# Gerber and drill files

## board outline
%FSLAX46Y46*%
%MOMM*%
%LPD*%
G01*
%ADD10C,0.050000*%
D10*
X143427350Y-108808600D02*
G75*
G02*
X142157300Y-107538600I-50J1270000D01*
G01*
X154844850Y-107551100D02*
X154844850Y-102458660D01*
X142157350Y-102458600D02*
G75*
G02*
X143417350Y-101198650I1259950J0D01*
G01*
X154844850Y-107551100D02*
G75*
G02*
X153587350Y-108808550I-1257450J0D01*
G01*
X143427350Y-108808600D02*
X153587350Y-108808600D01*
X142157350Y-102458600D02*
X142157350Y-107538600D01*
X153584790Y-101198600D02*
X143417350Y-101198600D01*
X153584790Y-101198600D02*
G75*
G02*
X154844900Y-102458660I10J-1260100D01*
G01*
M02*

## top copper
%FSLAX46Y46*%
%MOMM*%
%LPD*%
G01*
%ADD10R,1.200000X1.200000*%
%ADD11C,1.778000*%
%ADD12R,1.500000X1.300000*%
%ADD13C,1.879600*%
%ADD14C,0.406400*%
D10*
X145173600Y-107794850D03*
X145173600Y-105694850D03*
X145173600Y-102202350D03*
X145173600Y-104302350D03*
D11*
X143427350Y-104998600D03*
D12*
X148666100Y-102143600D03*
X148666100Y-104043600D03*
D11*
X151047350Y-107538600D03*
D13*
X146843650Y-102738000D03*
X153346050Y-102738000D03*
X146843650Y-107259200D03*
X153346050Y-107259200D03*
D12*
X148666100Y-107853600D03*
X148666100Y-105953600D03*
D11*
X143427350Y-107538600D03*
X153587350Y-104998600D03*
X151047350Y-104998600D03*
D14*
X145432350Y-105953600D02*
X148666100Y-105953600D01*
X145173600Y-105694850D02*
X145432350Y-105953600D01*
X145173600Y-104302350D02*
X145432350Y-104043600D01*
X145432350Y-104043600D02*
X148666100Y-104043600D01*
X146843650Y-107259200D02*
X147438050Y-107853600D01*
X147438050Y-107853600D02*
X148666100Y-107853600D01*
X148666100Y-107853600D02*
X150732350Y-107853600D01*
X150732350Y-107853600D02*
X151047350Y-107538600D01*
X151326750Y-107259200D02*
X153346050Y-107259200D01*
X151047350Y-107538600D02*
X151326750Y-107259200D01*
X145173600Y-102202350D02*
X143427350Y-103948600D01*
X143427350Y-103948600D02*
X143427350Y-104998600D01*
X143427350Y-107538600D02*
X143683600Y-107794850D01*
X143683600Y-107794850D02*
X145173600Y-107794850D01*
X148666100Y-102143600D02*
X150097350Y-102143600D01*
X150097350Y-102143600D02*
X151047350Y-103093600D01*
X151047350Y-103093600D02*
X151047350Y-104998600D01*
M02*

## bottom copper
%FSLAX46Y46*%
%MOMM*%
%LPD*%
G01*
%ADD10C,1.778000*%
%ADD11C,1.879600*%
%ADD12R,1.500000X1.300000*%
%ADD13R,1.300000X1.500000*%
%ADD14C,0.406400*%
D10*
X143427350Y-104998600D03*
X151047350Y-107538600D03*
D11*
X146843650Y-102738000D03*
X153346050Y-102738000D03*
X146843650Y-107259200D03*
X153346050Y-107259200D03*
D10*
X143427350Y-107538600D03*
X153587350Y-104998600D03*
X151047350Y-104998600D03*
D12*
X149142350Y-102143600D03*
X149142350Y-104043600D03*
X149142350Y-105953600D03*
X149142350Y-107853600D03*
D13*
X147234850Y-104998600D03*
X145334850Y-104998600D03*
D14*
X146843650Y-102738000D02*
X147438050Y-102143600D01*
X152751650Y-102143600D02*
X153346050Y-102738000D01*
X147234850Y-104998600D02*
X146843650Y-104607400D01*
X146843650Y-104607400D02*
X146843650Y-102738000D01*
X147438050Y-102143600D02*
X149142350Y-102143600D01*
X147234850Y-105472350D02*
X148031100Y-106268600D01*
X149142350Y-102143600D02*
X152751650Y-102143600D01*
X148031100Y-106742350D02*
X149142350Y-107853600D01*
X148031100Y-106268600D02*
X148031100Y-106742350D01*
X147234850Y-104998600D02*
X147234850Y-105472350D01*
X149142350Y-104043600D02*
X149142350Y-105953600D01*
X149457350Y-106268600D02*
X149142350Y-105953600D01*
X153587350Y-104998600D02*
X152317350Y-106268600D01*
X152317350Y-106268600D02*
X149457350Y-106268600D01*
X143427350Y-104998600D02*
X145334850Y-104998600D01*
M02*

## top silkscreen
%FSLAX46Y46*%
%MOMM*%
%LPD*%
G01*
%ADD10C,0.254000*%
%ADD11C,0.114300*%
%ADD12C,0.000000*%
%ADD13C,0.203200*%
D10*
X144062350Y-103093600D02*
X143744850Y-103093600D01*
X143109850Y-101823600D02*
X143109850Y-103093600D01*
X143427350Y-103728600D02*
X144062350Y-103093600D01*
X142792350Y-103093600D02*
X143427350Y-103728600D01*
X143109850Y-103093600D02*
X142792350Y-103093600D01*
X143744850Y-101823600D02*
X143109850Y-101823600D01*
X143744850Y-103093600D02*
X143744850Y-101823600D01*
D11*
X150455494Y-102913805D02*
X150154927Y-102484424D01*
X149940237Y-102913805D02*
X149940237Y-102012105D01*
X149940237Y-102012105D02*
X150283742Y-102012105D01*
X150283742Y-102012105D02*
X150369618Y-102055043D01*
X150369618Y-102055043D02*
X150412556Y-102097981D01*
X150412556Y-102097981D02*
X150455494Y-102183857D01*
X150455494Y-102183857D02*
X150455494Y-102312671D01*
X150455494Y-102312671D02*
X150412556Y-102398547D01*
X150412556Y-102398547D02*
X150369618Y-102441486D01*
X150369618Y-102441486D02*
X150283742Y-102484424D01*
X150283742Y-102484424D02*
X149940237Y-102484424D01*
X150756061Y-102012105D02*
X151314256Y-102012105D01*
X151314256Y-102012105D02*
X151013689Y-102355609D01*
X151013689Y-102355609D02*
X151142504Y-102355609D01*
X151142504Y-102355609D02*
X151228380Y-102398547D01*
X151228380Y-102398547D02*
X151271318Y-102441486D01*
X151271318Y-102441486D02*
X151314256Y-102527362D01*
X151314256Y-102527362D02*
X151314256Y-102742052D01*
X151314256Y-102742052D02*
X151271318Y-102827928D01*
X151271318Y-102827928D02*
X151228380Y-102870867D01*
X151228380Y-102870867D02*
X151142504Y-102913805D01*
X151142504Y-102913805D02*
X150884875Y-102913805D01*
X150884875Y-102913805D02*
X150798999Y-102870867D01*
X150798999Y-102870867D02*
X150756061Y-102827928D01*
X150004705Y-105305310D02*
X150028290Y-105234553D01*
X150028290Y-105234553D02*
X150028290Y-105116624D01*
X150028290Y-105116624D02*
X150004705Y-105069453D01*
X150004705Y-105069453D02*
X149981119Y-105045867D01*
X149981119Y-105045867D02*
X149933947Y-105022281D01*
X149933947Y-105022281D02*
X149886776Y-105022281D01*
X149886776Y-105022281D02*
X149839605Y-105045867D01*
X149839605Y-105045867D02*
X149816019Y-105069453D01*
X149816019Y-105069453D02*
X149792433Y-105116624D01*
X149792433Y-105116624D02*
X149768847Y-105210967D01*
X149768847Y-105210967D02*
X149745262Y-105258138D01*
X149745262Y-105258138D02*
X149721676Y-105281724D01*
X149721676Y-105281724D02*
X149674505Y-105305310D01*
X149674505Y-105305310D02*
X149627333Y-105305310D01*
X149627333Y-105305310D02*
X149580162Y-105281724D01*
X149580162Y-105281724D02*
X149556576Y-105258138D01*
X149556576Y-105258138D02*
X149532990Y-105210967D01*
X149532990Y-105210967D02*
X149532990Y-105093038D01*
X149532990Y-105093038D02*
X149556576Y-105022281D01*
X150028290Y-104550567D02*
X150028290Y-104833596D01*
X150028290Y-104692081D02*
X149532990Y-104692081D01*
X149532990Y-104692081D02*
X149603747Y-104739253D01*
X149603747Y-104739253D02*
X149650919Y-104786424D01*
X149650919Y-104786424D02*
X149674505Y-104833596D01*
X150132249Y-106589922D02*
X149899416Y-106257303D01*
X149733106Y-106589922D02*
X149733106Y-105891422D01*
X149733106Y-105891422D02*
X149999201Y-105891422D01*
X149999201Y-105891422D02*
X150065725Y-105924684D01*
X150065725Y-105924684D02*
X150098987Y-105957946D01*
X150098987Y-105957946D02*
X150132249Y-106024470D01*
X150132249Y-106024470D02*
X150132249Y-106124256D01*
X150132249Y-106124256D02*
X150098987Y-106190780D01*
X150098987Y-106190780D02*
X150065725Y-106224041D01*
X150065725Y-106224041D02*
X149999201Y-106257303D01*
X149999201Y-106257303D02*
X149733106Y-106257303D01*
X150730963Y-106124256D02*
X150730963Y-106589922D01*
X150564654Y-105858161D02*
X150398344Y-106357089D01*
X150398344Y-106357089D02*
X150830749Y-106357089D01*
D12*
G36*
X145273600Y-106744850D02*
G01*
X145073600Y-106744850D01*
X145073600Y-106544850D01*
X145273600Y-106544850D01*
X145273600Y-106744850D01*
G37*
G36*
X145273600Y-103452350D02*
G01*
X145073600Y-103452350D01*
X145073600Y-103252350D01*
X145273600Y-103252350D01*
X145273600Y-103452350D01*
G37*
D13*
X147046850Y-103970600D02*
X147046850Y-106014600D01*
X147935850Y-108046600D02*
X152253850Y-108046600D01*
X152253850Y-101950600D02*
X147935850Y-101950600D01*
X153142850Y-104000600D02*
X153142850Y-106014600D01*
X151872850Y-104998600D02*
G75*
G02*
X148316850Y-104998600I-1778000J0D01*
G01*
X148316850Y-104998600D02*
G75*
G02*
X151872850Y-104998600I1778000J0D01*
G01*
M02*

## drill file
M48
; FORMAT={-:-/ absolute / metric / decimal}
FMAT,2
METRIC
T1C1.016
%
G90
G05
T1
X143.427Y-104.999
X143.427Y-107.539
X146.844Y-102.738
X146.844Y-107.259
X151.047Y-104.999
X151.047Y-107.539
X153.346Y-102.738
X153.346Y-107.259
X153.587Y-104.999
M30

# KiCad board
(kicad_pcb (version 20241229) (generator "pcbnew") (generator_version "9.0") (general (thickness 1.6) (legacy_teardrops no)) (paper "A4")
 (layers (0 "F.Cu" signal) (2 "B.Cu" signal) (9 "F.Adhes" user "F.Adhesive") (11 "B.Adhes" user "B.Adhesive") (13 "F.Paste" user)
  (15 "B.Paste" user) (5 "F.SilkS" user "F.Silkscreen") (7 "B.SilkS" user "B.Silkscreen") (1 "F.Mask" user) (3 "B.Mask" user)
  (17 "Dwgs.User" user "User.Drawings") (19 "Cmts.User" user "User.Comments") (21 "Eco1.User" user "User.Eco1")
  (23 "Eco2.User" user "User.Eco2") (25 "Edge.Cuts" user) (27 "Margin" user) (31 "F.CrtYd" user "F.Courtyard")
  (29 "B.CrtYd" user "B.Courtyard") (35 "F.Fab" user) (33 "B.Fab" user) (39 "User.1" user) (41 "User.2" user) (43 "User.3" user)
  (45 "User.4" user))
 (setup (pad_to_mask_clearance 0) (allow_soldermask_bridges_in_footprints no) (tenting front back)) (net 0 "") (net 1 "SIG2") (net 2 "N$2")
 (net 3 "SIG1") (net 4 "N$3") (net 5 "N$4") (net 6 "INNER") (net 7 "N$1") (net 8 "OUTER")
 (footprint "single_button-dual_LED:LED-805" (layer "F.Cu") (at 145.1736 106.74485)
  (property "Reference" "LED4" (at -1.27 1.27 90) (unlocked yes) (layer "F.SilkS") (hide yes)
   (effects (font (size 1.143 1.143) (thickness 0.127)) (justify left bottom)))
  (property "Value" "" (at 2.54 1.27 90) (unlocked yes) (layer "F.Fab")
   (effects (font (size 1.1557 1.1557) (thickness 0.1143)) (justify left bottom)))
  (fp_poly (pts (xy -0.1 0) (xy 0.1 0) (xy 0.1 -0.2) (xy -0.1 -0.2)) (stroke (width 0) (type default)) (fill yes) (layer "F.SilkS"))
  (pad "A" smd rect (at 0 1.05) (size 1.2 1.2) (layers "F.Cu" "F.Mask" "F.Paste") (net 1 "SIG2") (solder_mask_margin 0.0508)
   (solder_paste_margin 0) (thermal_bridge_angle 0))
  (pad "C" smd rect (at 0 -1.05) (size 1.2 1.2) (layers "F.Cu" "F.Mask" "F.Paste") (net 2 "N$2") (solder_mask_margin 0.0508)
   (solder_paste_margin 0) (thermal_bridge_angle 0)))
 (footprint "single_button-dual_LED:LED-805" (layer "F.Cu") (at 145.1736 103.25235 180)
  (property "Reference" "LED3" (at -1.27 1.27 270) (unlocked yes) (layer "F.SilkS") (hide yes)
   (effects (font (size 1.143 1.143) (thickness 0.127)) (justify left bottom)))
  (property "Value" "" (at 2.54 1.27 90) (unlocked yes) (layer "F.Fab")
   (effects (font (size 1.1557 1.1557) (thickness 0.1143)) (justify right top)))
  (fp_poly (pts (xy -0.1 0) (xy 0.1 0) (xy 0.1 -0.2) (xy -0.1 -0.2)) (stroke (width 0) (type default)) (fill yes) (layer "F.SilkS"))
  (pad "A" smd rect (at 0 1.05 180) (size 1.2 1.2) (layers "F.Cu" "F.Mask" "F.Paste") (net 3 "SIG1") (solder_mask_margin 0.0508)
   (solder_paste_margin 0) (thermal_bridge_angle 0))
  (pad "C" smd rect (at 0 -1.05 180) (size 1.2 1.2) (layers "F.Cu" "F.Mask" "F.Paste") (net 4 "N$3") (solder_mask_margin 0.0508)
   (solder_paste_margin 0) (thermal_bridge_angle 0)))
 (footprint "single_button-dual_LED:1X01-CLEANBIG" (layer "F.Cu") (at 143.42735 104.9986)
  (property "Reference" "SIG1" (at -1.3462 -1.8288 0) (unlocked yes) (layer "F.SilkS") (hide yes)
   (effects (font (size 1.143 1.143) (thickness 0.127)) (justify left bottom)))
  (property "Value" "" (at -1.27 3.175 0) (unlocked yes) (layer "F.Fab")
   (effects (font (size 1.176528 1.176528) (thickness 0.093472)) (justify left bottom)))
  (pad "1" thru_hole circle (at 0 0) (size 1.778 1.778) (drill 1.016) (layers "*.Cu" "*.Mask") (remove_unused_layers no) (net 3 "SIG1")
   (solder_mask_margin 0.0508) (thermal_bridge_angle 0)))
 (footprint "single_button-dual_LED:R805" (layer "F.Cu") (at 148.6661 103.0936 -90)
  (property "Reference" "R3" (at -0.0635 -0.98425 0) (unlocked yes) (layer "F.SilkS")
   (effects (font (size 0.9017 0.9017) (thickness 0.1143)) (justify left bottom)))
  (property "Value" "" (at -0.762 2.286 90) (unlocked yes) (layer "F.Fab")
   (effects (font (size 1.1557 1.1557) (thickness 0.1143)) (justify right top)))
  (pad "1" smd rect (at -0.95 0 270) (size 1.3 1.5) (layers "F.Cu" "F.Mask" "F.Paste") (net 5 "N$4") (solder_mask_margin 0.0508)
   (solder_paste_margin 0) (thermal_bridge_angle 0))
  (pad "2" smd rect (at 0.95 0 270) (size 1.3 1.5) (layers "F.Cu" "F.Mask" "F.Paste") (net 4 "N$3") (solder_mask_margin 0.0508)
   (solder_paste_margin 0) (thermal_bridge_angle 0)))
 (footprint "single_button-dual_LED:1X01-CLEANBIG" (layer "F.Cu") (at 151.04735 107.5386)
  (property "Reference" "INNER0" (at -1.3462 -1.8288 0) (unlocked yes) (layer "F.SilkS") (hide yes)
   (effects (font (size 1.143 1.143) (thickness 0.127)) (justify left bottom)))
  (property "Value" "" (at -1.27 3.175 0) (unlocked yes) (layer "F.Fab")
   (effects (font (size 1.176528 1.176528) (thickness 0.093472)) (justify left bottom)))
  (pad "1" thru_hole circle (at 0 0) (size 1.778 1.778) (drill 1.016) (layers "*.Cu" "*.Mask") (remove_unused_layers no) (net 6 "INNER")
   (solder_mask_margin 0.0508) (thermal_bridge_angle 0)))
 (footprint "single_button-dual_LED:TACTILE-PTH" (layer "F.Cu") (at 150.09485 104.9986)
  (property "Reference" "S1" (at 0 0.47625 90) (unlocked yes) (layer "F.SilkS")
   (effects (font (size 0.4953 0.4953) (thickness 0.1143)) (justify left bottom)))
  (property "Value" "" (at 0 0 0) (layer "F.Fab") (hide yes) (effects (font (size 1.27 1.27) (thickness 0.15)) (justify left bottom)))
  (fp_line (start -3.048 -1.028) (end -3.048 1.016) (stroke (width 0.2032) (type solid)) (layer "F.SilkS"))
  (fp_line (start -2.159 3.048) (end 2.159 3.048) (stroke (width 0.2032) (type solid)) (layer "F.SilkS"))
  (fp_line (start 2.159 -3.048) (end -2.159 -3.048) (stroke (width 0.2032) (type solid)) (layer "F.SilkS"))
  (fp_line (start 3.048 -0.998) (end 3.048 1.016) (stroke (width 0.2032) (type solid)) (layer "F.SilkS"))
  (fp_circle (center 0 0) (end 1.778 0) (stroke (width 0.2032) (type solid)) (fill no) (layer "F.SilkS"))
  (pad "1" thru_hole circle (at -3.2512 -2.2606) (size 1.8796 1.8796) (drill 1.016) (layers "*.Cu" "*.Mask") (remove_unused_layers no)
   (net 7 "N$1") (solder_mask_margin 0.0508) (thermal_bridge_angle 0))
  (pad "2" thru_hole circle (at 3.2512 -2.2606) (size 1.8796 1.8796) (drill 1.016) (layers "*.Cu" "*.Mask") (remove_unused_layers no)
   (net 7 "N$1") (solder_mask_margin 0.0508) (thermal_bridge_angle 0))
  (pad "3" thru_hole circle (at -3.2512 2.2606) (size 1.8796 1.8796) (drill 1.016) (layers "*.Cu" "*.Mask") (remove_unused_layers no)
   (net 6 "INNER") (solder_mask_margin 0.0508) (thermal_bridge_angle 0))
  (pad "4" thru_hole circle (at 3.2512 2.2606) (size 1.8796 1.8796) (drill 1.016) (layers "*.Cu" "*.Mask") (remove_unused_layers no)
   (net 6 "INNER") (solder_mask_margin 0.0508) (thermal_bridge_angle 0)))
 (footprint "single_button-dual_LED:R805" (layer "F.Cu") (at 148.6661 106.9036 90)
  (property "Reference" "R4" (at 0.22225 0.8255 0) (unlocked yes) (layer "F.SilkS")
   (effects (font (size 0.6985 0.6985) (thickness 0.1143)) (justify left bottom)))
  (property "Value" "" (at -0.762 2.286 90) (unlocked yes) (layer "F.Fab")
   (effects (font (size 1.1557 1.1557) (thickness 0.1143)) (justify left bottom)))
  (pad "1" smd rect (at -0.95 0 90) (size 1.3 1.5) (layers "F.Cu" "F.Mask" "F.Paste") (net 6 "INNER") (solder_mask_margin 0.0508)
   (solder_paste_margin 0) (thermal_bridge_angle 0))
  (pad "2" smd rect (at 0.95 0 90) (size 1.3 1.5) (layers "F.Cu" "F.Mask" "F.Paste") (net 2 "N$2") (solder_mask_margin 0.0508)
   (solder_paste_margin 0) (thermal_bridge_angle 0)))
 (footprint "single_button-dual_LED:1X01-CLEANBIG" (layer "F.Cu") (at 143.42735 107.5386)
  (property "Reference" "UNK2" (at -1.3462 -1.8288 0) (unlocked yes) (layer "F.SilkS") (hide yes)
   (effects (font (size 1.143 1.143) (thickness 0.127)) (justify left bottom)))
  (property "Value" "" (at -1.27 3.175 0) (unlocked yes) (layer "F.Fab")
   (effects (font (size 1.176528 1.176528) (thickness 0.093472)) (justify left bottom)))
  (pad "1" thru_hole circle (at 0 0) (size 1.778 1.778) (drill 1.016) (layers "*.Cu" "*.Mask") (remove_unused_layers no) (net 1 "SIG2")
   (solder_mask_margin 0.0508) (thermal_bridge_angle 0)))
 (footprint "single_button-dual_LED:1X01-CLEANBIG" (layer "F.Cu") (at 153.58735 104.9986)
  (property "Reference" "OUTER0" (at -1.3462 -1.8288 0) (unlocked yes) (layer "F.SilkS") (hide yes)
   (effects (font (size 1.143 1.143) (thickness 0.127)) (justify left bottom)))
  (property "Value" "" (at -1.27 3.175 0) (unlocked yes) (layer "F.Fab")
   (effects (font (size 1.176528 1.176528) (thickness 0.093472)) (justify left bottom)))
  (pad "1" thru_hole circle (at 0 0) (size 1.778 1.778) (drill 1.016) (layers "*.Cu" "*.Mask") (remove_unused_layers no) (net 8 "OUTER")
   (solder_mask_margin 0.0508) (thermal_bridge_angle 0)))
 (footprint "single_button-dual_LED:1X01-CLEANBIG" (layer "F.Cu") (at 151.04735 104.9986)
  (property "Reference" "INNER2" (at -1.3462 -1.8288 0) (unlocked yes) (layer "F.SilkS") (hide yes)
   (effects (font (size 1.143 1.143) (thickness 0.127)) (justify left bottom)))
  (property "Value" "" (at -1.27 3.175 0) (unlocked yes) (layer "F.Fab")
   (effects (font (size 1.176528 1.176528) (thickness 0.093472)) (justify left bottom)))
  (pad "1" thru_hole circle (at 0 0) (size 1.778 1.778) (drill 1.016) (layers "*.Cu" "*.Mask") (remove_unused_layers no) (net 5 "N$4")
   (solder_mask_margin 0.0508) (thermal_bridge_angle 0)))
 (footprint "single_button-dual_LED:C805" (layer "B.Cu") (at 149.14235 103.0936 -90)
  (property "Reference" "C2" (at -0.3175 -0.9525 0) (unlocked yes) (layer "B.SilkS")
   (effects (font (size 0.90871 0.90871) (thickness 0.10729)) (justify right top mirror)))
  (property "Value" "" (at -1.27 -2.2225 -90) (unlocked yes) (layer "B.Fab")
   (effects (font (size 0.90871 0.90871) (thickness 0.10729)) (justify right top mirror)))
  (pad "1" smd rect (at -0.95 0 270) (size 1.3 1.5) (layers "B.Cu" "B.Mask" "B.Paste") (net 7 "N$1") (solder_mask_margin 0.0508)
   (solder_paste_margin 0) (thermal_bridge_angle 0))
  (pad "2" smd rect (at 0.95 0 270) (size 1.3 1.5) (layers "B.Cu" "B.Mask" "B.Paste") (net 8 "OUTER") (solder_mask_margin 0.0508)
   (solder_paste_margin 0) (thermal_bridge_angle 0)))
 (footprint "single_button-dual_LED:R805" (layer "B.Cu") (at 149.14235 106.9036 -90)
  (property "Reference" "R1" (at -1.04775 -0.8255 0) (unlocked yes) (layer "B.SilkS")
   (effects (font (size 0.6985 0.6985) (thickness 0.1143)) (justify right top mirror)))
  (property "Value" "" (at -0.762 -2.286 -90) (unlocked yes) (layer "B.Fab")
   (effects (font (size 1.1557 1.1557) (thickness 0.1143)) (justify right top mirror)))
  (pad "1" smd rect (at -0.95 0 270) (size 1.3 1.5) (layers "B.Cu" "B.Mask" "B.Paste") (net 8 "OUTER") (solder_mask_margin 0.0508)
   (solder_paste_margin 0) (thermal_bridge_angle 0))
  (pad "2" smd rect (at 0.95 0 270) (size 1.3 1.5) (layers "B.Cu" "B.Mask" "B.Paste") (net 7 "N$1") (solder_mask_margin 0.0508)
   (solder_paste_margin 0) (thermal_bridge_angle 0)))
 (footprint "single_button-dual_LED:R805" (layer "B.Cu") (at 146.28485 104.9986 180)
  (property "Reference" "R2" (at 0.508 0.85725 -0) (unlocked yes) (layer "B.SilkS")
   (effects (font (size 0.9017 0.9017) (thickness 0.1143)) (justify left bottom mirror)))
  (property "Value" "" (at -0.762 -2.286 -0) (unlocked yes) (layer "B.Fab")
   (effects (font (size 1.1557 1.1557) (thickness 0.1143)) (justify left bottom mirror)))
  (pad "1" smd rect (at -0.95 0 180) (size 1.3 1.5) (layers "B.Cu" "B.Mask" "B.Paste") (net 7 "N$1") (solder_mask_margin 0.0508)
   (solder_paste_margin 0) (thermal_bridge_angle 0))
  (pad "2" smd rect (at 0.95 0 180) (size 1.3 1.5) (layers "B.Cu" "B.Mask" "B.Paste") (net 3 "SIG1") (solder_mask_margin 0.0508)
   (solder_paste_margin 0) (thermal_bridge_angle 0)))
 (gr_line (start 144.06235 103.0936) (end 143.74485 103.0936) (stroke (width 0.254) (type solid)) (layer "F.SilkS"))
 (gr_line (start 143.10985 101.8236) (end 143.10985 103.0936) (stroke (width 0.254) (type solid)) (layer "F.SilkS"))
 (gr_line (start 143.42735 103.7286) (end 144.06235 103.0936) (stroke (width 0.254) (type solid)) (layer "F.SilkS"))
 (gr_line (start 142.79235 103.0936) (end 143.42735 103.7286) (stroke (width 0.254) (type solid)) (layer "F.SilkS"))
 (gr_line (start 143.10985 103.0936) (end 142.79235 103.0936) (stroke (width 0.254) (type solid)) (layer "F.SilkS"))
 (gr_line (start 143.74485 101.8236) (end 143.10985 101.8236) (stroke (width 0.254) (type solid)) (layer "F.SilkS"))
 (gr_line (start 143.74485 103.0936) (end 143.74485 101.8236) (stroke (width 0.254) (type solid)) (layer "F.SilkS"))
 (gr_arc (start 143.42735 108.8086) (mid 142.529324 108.436626) (end 142.15735 107.5386) (stroke (width 0.05) (type solid))
  (layer "Edge.Cuts"))
 (gr_line (start 154.84485 107.5511) (end 154.84485 102.45866) (stroke (width 0.05) (type solid)) (layer "Edge.Cuts"))
 (gr_arc (start 142.15735 102.4586) (mid 142.526395 101.567645) (end 143.41735 101.1986) (stroke (width 0.05) (type solid))
  (layer "Edge.Cuts"))
 (gr_arc (start 154.84485 107.5511) (mid 154.476537 108.440287) (end 153.58735 108.8086) (stroke (width 0.05) (type solid))
  (layer "Edge.Cuts"))
 (gr_line (start 143.42735 108.8086) (end 153.58735 108.8086) (stroke (width 0.05) (type solid)) (layer "Edge.Cuts"))
 (gr_line (start 142.15735 102.4586) (end 142.15735 107.5386) (stroke (width 0.05) (type solid)) (layer "Edge.Cuts"))
 (gr_line (start 153.58479 101.1986) (end 143.41735 101.1986) (stroke (width 0.05) (type solid)) (layer "Edge.Cuts"))
 (gr_arc (start 153.58479 101.1986) (mid 154.475787 101.567663) (end 154.84485 102.45866) (stroke (width 0.05) (type solid))
  (layer "Edge.Cuts"))
 (segment (start 146.84365 102.738) (end 147.43805 102.1436) (width 0.4064) (layer "B.Cu") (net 7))
 (segment (start 152.75165 102.1436) (end 153.34605 102.738) (width 0.4064) (layer "B.Cu") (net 7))
 (segment (start 147.23485 104.9986) (end 146.84365 104.6074) (width 0.4064) (layer "B.Cu") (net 7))
 (segment (start 146.84365 104.6074) (end 146.84365 102.738) (width 0.4064) (layer "B.Cu") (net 7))
 (segment (start 147.43805 102.1436) (end 149.14235 102.1436) (width 0.4064) (layer "B.Cu") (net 7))
 (segment (start 147.23485 105.47235) (end 148.0311 106.2686) (width 0.4064) (layer "B.Cu") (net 7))
 (segment (start 149.14235 102.1436) (end 152.75165 102.1436) (width 0.4064) (layer "B.Cu") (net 7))
 (segment (start 148.0311 106.74235) (end 149.14235 107.8536) (width 0.4064) (layer "B.Cu") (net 7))
 (segment (start 148.0311 106.2686) (end 148.0311 106.74235) (width 0.4064) (layer "B.Cu") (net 7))
 (segment (start 147.23485 104.9986) (end 147.23485 105.47235) (width 0.4064) (layer "B.Cu") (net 7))
 (segment (start 149.14235 104.0436) (end 149.14235 105.9536) (width 0.4064) (layer "B.Cu") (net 8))
 (segment (start 149.45735 106.2686) (end 149.14235 105.9536) (width 0.4064) (layer "B.Cu") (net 8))
 (segment (start 153.58735 104.9986) (end 152.31735 106.2686) (width 0.4064) (layer "B.Cu") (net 8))
 (segment (start 152.31735 106.2686) (end 149.45735 106.2686) (width 0.4064) (layer "B.Cu") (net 8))
 (segment (start 145.43235 105.9536) (end 148.6661 105.9536) (width 0.4064) (layer "F.Cu") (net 2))
 (segment (start 145.1736 105.69485) (end 145.43235 105.9536) (width 0.4064) (layer "F.Cu") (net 2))
 (segment (start 145.1736 104.30235) (end 145.43235 104.0436) (width 0.4064) (layer "F.Cu") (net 4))
 (segment (start 145.43235 104.0436) (end 148.6661 104.0436) (width 0.4064) (layer "F.Cu") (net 4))
 (segment (start 146.84365 107.2592) (end 147.43805 107.8536) (width 0.4064) (layer "F.Cu") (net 6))
 (segment (start 147.43805 107.8536) (end 148.6661 107.8536) (width 0.4064) (layer "F.Cu") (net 6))
 (segment (start 148.6661 107.8536) (end 150.73235 107.8536) (width 0.4064) (layer "F.Cu") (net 6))
 (segment (start 150.73235 107.8536) (end 151.04735 107.5386) (width 0.4064) (layer "F.Cu") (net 6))
 (segment (start 151.32675 107.2592) (end 153.34605 107.2592) (width 0.4064) (layer "F.Cu") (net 6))
 (segment (start 151.04735 107.5386) (end 151.32675 107.2592) (width 0.4064) (layer "F.Cu") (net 6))
 (segment (start 145.1736 102.20235) (end 143.42735 103.9486) (width 0.4064) (layer "F.Cu") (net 3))
 (segment (start 143.42735 103.9486) (end 143.42735 104.9986) (width 0.4064) (layer "F.Cu") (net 3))
 (segment (start 143.42735 104.9986) (end 145.33485 104.9986) (width 0.4064) (layer "B.Cu") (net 3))
 (segment (start 143.42735 107.5386) (end 143.6836 107.79485) (width 0.4064) (layer "F.Cu") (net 1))
 (segment (start 143.6836 107.79485) (end 145.1736 107.79485) (width 0.4064) (layer "F.Cu") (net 1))
 (segment (start 148.6661 102.1436) (end 150.09735 102.1436) (width 0.4064) (layer "F.Cu") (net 5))
 (segment (start 150.09735 102.1436) (end 151.04735 103.0936) (width 0.4064) (layer "F.Cu") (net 5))
 (segment (start 151.04735 103.0936) (end 151.04735 104.9986) (width 0.4064) (layer "F.Cu") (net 5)))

